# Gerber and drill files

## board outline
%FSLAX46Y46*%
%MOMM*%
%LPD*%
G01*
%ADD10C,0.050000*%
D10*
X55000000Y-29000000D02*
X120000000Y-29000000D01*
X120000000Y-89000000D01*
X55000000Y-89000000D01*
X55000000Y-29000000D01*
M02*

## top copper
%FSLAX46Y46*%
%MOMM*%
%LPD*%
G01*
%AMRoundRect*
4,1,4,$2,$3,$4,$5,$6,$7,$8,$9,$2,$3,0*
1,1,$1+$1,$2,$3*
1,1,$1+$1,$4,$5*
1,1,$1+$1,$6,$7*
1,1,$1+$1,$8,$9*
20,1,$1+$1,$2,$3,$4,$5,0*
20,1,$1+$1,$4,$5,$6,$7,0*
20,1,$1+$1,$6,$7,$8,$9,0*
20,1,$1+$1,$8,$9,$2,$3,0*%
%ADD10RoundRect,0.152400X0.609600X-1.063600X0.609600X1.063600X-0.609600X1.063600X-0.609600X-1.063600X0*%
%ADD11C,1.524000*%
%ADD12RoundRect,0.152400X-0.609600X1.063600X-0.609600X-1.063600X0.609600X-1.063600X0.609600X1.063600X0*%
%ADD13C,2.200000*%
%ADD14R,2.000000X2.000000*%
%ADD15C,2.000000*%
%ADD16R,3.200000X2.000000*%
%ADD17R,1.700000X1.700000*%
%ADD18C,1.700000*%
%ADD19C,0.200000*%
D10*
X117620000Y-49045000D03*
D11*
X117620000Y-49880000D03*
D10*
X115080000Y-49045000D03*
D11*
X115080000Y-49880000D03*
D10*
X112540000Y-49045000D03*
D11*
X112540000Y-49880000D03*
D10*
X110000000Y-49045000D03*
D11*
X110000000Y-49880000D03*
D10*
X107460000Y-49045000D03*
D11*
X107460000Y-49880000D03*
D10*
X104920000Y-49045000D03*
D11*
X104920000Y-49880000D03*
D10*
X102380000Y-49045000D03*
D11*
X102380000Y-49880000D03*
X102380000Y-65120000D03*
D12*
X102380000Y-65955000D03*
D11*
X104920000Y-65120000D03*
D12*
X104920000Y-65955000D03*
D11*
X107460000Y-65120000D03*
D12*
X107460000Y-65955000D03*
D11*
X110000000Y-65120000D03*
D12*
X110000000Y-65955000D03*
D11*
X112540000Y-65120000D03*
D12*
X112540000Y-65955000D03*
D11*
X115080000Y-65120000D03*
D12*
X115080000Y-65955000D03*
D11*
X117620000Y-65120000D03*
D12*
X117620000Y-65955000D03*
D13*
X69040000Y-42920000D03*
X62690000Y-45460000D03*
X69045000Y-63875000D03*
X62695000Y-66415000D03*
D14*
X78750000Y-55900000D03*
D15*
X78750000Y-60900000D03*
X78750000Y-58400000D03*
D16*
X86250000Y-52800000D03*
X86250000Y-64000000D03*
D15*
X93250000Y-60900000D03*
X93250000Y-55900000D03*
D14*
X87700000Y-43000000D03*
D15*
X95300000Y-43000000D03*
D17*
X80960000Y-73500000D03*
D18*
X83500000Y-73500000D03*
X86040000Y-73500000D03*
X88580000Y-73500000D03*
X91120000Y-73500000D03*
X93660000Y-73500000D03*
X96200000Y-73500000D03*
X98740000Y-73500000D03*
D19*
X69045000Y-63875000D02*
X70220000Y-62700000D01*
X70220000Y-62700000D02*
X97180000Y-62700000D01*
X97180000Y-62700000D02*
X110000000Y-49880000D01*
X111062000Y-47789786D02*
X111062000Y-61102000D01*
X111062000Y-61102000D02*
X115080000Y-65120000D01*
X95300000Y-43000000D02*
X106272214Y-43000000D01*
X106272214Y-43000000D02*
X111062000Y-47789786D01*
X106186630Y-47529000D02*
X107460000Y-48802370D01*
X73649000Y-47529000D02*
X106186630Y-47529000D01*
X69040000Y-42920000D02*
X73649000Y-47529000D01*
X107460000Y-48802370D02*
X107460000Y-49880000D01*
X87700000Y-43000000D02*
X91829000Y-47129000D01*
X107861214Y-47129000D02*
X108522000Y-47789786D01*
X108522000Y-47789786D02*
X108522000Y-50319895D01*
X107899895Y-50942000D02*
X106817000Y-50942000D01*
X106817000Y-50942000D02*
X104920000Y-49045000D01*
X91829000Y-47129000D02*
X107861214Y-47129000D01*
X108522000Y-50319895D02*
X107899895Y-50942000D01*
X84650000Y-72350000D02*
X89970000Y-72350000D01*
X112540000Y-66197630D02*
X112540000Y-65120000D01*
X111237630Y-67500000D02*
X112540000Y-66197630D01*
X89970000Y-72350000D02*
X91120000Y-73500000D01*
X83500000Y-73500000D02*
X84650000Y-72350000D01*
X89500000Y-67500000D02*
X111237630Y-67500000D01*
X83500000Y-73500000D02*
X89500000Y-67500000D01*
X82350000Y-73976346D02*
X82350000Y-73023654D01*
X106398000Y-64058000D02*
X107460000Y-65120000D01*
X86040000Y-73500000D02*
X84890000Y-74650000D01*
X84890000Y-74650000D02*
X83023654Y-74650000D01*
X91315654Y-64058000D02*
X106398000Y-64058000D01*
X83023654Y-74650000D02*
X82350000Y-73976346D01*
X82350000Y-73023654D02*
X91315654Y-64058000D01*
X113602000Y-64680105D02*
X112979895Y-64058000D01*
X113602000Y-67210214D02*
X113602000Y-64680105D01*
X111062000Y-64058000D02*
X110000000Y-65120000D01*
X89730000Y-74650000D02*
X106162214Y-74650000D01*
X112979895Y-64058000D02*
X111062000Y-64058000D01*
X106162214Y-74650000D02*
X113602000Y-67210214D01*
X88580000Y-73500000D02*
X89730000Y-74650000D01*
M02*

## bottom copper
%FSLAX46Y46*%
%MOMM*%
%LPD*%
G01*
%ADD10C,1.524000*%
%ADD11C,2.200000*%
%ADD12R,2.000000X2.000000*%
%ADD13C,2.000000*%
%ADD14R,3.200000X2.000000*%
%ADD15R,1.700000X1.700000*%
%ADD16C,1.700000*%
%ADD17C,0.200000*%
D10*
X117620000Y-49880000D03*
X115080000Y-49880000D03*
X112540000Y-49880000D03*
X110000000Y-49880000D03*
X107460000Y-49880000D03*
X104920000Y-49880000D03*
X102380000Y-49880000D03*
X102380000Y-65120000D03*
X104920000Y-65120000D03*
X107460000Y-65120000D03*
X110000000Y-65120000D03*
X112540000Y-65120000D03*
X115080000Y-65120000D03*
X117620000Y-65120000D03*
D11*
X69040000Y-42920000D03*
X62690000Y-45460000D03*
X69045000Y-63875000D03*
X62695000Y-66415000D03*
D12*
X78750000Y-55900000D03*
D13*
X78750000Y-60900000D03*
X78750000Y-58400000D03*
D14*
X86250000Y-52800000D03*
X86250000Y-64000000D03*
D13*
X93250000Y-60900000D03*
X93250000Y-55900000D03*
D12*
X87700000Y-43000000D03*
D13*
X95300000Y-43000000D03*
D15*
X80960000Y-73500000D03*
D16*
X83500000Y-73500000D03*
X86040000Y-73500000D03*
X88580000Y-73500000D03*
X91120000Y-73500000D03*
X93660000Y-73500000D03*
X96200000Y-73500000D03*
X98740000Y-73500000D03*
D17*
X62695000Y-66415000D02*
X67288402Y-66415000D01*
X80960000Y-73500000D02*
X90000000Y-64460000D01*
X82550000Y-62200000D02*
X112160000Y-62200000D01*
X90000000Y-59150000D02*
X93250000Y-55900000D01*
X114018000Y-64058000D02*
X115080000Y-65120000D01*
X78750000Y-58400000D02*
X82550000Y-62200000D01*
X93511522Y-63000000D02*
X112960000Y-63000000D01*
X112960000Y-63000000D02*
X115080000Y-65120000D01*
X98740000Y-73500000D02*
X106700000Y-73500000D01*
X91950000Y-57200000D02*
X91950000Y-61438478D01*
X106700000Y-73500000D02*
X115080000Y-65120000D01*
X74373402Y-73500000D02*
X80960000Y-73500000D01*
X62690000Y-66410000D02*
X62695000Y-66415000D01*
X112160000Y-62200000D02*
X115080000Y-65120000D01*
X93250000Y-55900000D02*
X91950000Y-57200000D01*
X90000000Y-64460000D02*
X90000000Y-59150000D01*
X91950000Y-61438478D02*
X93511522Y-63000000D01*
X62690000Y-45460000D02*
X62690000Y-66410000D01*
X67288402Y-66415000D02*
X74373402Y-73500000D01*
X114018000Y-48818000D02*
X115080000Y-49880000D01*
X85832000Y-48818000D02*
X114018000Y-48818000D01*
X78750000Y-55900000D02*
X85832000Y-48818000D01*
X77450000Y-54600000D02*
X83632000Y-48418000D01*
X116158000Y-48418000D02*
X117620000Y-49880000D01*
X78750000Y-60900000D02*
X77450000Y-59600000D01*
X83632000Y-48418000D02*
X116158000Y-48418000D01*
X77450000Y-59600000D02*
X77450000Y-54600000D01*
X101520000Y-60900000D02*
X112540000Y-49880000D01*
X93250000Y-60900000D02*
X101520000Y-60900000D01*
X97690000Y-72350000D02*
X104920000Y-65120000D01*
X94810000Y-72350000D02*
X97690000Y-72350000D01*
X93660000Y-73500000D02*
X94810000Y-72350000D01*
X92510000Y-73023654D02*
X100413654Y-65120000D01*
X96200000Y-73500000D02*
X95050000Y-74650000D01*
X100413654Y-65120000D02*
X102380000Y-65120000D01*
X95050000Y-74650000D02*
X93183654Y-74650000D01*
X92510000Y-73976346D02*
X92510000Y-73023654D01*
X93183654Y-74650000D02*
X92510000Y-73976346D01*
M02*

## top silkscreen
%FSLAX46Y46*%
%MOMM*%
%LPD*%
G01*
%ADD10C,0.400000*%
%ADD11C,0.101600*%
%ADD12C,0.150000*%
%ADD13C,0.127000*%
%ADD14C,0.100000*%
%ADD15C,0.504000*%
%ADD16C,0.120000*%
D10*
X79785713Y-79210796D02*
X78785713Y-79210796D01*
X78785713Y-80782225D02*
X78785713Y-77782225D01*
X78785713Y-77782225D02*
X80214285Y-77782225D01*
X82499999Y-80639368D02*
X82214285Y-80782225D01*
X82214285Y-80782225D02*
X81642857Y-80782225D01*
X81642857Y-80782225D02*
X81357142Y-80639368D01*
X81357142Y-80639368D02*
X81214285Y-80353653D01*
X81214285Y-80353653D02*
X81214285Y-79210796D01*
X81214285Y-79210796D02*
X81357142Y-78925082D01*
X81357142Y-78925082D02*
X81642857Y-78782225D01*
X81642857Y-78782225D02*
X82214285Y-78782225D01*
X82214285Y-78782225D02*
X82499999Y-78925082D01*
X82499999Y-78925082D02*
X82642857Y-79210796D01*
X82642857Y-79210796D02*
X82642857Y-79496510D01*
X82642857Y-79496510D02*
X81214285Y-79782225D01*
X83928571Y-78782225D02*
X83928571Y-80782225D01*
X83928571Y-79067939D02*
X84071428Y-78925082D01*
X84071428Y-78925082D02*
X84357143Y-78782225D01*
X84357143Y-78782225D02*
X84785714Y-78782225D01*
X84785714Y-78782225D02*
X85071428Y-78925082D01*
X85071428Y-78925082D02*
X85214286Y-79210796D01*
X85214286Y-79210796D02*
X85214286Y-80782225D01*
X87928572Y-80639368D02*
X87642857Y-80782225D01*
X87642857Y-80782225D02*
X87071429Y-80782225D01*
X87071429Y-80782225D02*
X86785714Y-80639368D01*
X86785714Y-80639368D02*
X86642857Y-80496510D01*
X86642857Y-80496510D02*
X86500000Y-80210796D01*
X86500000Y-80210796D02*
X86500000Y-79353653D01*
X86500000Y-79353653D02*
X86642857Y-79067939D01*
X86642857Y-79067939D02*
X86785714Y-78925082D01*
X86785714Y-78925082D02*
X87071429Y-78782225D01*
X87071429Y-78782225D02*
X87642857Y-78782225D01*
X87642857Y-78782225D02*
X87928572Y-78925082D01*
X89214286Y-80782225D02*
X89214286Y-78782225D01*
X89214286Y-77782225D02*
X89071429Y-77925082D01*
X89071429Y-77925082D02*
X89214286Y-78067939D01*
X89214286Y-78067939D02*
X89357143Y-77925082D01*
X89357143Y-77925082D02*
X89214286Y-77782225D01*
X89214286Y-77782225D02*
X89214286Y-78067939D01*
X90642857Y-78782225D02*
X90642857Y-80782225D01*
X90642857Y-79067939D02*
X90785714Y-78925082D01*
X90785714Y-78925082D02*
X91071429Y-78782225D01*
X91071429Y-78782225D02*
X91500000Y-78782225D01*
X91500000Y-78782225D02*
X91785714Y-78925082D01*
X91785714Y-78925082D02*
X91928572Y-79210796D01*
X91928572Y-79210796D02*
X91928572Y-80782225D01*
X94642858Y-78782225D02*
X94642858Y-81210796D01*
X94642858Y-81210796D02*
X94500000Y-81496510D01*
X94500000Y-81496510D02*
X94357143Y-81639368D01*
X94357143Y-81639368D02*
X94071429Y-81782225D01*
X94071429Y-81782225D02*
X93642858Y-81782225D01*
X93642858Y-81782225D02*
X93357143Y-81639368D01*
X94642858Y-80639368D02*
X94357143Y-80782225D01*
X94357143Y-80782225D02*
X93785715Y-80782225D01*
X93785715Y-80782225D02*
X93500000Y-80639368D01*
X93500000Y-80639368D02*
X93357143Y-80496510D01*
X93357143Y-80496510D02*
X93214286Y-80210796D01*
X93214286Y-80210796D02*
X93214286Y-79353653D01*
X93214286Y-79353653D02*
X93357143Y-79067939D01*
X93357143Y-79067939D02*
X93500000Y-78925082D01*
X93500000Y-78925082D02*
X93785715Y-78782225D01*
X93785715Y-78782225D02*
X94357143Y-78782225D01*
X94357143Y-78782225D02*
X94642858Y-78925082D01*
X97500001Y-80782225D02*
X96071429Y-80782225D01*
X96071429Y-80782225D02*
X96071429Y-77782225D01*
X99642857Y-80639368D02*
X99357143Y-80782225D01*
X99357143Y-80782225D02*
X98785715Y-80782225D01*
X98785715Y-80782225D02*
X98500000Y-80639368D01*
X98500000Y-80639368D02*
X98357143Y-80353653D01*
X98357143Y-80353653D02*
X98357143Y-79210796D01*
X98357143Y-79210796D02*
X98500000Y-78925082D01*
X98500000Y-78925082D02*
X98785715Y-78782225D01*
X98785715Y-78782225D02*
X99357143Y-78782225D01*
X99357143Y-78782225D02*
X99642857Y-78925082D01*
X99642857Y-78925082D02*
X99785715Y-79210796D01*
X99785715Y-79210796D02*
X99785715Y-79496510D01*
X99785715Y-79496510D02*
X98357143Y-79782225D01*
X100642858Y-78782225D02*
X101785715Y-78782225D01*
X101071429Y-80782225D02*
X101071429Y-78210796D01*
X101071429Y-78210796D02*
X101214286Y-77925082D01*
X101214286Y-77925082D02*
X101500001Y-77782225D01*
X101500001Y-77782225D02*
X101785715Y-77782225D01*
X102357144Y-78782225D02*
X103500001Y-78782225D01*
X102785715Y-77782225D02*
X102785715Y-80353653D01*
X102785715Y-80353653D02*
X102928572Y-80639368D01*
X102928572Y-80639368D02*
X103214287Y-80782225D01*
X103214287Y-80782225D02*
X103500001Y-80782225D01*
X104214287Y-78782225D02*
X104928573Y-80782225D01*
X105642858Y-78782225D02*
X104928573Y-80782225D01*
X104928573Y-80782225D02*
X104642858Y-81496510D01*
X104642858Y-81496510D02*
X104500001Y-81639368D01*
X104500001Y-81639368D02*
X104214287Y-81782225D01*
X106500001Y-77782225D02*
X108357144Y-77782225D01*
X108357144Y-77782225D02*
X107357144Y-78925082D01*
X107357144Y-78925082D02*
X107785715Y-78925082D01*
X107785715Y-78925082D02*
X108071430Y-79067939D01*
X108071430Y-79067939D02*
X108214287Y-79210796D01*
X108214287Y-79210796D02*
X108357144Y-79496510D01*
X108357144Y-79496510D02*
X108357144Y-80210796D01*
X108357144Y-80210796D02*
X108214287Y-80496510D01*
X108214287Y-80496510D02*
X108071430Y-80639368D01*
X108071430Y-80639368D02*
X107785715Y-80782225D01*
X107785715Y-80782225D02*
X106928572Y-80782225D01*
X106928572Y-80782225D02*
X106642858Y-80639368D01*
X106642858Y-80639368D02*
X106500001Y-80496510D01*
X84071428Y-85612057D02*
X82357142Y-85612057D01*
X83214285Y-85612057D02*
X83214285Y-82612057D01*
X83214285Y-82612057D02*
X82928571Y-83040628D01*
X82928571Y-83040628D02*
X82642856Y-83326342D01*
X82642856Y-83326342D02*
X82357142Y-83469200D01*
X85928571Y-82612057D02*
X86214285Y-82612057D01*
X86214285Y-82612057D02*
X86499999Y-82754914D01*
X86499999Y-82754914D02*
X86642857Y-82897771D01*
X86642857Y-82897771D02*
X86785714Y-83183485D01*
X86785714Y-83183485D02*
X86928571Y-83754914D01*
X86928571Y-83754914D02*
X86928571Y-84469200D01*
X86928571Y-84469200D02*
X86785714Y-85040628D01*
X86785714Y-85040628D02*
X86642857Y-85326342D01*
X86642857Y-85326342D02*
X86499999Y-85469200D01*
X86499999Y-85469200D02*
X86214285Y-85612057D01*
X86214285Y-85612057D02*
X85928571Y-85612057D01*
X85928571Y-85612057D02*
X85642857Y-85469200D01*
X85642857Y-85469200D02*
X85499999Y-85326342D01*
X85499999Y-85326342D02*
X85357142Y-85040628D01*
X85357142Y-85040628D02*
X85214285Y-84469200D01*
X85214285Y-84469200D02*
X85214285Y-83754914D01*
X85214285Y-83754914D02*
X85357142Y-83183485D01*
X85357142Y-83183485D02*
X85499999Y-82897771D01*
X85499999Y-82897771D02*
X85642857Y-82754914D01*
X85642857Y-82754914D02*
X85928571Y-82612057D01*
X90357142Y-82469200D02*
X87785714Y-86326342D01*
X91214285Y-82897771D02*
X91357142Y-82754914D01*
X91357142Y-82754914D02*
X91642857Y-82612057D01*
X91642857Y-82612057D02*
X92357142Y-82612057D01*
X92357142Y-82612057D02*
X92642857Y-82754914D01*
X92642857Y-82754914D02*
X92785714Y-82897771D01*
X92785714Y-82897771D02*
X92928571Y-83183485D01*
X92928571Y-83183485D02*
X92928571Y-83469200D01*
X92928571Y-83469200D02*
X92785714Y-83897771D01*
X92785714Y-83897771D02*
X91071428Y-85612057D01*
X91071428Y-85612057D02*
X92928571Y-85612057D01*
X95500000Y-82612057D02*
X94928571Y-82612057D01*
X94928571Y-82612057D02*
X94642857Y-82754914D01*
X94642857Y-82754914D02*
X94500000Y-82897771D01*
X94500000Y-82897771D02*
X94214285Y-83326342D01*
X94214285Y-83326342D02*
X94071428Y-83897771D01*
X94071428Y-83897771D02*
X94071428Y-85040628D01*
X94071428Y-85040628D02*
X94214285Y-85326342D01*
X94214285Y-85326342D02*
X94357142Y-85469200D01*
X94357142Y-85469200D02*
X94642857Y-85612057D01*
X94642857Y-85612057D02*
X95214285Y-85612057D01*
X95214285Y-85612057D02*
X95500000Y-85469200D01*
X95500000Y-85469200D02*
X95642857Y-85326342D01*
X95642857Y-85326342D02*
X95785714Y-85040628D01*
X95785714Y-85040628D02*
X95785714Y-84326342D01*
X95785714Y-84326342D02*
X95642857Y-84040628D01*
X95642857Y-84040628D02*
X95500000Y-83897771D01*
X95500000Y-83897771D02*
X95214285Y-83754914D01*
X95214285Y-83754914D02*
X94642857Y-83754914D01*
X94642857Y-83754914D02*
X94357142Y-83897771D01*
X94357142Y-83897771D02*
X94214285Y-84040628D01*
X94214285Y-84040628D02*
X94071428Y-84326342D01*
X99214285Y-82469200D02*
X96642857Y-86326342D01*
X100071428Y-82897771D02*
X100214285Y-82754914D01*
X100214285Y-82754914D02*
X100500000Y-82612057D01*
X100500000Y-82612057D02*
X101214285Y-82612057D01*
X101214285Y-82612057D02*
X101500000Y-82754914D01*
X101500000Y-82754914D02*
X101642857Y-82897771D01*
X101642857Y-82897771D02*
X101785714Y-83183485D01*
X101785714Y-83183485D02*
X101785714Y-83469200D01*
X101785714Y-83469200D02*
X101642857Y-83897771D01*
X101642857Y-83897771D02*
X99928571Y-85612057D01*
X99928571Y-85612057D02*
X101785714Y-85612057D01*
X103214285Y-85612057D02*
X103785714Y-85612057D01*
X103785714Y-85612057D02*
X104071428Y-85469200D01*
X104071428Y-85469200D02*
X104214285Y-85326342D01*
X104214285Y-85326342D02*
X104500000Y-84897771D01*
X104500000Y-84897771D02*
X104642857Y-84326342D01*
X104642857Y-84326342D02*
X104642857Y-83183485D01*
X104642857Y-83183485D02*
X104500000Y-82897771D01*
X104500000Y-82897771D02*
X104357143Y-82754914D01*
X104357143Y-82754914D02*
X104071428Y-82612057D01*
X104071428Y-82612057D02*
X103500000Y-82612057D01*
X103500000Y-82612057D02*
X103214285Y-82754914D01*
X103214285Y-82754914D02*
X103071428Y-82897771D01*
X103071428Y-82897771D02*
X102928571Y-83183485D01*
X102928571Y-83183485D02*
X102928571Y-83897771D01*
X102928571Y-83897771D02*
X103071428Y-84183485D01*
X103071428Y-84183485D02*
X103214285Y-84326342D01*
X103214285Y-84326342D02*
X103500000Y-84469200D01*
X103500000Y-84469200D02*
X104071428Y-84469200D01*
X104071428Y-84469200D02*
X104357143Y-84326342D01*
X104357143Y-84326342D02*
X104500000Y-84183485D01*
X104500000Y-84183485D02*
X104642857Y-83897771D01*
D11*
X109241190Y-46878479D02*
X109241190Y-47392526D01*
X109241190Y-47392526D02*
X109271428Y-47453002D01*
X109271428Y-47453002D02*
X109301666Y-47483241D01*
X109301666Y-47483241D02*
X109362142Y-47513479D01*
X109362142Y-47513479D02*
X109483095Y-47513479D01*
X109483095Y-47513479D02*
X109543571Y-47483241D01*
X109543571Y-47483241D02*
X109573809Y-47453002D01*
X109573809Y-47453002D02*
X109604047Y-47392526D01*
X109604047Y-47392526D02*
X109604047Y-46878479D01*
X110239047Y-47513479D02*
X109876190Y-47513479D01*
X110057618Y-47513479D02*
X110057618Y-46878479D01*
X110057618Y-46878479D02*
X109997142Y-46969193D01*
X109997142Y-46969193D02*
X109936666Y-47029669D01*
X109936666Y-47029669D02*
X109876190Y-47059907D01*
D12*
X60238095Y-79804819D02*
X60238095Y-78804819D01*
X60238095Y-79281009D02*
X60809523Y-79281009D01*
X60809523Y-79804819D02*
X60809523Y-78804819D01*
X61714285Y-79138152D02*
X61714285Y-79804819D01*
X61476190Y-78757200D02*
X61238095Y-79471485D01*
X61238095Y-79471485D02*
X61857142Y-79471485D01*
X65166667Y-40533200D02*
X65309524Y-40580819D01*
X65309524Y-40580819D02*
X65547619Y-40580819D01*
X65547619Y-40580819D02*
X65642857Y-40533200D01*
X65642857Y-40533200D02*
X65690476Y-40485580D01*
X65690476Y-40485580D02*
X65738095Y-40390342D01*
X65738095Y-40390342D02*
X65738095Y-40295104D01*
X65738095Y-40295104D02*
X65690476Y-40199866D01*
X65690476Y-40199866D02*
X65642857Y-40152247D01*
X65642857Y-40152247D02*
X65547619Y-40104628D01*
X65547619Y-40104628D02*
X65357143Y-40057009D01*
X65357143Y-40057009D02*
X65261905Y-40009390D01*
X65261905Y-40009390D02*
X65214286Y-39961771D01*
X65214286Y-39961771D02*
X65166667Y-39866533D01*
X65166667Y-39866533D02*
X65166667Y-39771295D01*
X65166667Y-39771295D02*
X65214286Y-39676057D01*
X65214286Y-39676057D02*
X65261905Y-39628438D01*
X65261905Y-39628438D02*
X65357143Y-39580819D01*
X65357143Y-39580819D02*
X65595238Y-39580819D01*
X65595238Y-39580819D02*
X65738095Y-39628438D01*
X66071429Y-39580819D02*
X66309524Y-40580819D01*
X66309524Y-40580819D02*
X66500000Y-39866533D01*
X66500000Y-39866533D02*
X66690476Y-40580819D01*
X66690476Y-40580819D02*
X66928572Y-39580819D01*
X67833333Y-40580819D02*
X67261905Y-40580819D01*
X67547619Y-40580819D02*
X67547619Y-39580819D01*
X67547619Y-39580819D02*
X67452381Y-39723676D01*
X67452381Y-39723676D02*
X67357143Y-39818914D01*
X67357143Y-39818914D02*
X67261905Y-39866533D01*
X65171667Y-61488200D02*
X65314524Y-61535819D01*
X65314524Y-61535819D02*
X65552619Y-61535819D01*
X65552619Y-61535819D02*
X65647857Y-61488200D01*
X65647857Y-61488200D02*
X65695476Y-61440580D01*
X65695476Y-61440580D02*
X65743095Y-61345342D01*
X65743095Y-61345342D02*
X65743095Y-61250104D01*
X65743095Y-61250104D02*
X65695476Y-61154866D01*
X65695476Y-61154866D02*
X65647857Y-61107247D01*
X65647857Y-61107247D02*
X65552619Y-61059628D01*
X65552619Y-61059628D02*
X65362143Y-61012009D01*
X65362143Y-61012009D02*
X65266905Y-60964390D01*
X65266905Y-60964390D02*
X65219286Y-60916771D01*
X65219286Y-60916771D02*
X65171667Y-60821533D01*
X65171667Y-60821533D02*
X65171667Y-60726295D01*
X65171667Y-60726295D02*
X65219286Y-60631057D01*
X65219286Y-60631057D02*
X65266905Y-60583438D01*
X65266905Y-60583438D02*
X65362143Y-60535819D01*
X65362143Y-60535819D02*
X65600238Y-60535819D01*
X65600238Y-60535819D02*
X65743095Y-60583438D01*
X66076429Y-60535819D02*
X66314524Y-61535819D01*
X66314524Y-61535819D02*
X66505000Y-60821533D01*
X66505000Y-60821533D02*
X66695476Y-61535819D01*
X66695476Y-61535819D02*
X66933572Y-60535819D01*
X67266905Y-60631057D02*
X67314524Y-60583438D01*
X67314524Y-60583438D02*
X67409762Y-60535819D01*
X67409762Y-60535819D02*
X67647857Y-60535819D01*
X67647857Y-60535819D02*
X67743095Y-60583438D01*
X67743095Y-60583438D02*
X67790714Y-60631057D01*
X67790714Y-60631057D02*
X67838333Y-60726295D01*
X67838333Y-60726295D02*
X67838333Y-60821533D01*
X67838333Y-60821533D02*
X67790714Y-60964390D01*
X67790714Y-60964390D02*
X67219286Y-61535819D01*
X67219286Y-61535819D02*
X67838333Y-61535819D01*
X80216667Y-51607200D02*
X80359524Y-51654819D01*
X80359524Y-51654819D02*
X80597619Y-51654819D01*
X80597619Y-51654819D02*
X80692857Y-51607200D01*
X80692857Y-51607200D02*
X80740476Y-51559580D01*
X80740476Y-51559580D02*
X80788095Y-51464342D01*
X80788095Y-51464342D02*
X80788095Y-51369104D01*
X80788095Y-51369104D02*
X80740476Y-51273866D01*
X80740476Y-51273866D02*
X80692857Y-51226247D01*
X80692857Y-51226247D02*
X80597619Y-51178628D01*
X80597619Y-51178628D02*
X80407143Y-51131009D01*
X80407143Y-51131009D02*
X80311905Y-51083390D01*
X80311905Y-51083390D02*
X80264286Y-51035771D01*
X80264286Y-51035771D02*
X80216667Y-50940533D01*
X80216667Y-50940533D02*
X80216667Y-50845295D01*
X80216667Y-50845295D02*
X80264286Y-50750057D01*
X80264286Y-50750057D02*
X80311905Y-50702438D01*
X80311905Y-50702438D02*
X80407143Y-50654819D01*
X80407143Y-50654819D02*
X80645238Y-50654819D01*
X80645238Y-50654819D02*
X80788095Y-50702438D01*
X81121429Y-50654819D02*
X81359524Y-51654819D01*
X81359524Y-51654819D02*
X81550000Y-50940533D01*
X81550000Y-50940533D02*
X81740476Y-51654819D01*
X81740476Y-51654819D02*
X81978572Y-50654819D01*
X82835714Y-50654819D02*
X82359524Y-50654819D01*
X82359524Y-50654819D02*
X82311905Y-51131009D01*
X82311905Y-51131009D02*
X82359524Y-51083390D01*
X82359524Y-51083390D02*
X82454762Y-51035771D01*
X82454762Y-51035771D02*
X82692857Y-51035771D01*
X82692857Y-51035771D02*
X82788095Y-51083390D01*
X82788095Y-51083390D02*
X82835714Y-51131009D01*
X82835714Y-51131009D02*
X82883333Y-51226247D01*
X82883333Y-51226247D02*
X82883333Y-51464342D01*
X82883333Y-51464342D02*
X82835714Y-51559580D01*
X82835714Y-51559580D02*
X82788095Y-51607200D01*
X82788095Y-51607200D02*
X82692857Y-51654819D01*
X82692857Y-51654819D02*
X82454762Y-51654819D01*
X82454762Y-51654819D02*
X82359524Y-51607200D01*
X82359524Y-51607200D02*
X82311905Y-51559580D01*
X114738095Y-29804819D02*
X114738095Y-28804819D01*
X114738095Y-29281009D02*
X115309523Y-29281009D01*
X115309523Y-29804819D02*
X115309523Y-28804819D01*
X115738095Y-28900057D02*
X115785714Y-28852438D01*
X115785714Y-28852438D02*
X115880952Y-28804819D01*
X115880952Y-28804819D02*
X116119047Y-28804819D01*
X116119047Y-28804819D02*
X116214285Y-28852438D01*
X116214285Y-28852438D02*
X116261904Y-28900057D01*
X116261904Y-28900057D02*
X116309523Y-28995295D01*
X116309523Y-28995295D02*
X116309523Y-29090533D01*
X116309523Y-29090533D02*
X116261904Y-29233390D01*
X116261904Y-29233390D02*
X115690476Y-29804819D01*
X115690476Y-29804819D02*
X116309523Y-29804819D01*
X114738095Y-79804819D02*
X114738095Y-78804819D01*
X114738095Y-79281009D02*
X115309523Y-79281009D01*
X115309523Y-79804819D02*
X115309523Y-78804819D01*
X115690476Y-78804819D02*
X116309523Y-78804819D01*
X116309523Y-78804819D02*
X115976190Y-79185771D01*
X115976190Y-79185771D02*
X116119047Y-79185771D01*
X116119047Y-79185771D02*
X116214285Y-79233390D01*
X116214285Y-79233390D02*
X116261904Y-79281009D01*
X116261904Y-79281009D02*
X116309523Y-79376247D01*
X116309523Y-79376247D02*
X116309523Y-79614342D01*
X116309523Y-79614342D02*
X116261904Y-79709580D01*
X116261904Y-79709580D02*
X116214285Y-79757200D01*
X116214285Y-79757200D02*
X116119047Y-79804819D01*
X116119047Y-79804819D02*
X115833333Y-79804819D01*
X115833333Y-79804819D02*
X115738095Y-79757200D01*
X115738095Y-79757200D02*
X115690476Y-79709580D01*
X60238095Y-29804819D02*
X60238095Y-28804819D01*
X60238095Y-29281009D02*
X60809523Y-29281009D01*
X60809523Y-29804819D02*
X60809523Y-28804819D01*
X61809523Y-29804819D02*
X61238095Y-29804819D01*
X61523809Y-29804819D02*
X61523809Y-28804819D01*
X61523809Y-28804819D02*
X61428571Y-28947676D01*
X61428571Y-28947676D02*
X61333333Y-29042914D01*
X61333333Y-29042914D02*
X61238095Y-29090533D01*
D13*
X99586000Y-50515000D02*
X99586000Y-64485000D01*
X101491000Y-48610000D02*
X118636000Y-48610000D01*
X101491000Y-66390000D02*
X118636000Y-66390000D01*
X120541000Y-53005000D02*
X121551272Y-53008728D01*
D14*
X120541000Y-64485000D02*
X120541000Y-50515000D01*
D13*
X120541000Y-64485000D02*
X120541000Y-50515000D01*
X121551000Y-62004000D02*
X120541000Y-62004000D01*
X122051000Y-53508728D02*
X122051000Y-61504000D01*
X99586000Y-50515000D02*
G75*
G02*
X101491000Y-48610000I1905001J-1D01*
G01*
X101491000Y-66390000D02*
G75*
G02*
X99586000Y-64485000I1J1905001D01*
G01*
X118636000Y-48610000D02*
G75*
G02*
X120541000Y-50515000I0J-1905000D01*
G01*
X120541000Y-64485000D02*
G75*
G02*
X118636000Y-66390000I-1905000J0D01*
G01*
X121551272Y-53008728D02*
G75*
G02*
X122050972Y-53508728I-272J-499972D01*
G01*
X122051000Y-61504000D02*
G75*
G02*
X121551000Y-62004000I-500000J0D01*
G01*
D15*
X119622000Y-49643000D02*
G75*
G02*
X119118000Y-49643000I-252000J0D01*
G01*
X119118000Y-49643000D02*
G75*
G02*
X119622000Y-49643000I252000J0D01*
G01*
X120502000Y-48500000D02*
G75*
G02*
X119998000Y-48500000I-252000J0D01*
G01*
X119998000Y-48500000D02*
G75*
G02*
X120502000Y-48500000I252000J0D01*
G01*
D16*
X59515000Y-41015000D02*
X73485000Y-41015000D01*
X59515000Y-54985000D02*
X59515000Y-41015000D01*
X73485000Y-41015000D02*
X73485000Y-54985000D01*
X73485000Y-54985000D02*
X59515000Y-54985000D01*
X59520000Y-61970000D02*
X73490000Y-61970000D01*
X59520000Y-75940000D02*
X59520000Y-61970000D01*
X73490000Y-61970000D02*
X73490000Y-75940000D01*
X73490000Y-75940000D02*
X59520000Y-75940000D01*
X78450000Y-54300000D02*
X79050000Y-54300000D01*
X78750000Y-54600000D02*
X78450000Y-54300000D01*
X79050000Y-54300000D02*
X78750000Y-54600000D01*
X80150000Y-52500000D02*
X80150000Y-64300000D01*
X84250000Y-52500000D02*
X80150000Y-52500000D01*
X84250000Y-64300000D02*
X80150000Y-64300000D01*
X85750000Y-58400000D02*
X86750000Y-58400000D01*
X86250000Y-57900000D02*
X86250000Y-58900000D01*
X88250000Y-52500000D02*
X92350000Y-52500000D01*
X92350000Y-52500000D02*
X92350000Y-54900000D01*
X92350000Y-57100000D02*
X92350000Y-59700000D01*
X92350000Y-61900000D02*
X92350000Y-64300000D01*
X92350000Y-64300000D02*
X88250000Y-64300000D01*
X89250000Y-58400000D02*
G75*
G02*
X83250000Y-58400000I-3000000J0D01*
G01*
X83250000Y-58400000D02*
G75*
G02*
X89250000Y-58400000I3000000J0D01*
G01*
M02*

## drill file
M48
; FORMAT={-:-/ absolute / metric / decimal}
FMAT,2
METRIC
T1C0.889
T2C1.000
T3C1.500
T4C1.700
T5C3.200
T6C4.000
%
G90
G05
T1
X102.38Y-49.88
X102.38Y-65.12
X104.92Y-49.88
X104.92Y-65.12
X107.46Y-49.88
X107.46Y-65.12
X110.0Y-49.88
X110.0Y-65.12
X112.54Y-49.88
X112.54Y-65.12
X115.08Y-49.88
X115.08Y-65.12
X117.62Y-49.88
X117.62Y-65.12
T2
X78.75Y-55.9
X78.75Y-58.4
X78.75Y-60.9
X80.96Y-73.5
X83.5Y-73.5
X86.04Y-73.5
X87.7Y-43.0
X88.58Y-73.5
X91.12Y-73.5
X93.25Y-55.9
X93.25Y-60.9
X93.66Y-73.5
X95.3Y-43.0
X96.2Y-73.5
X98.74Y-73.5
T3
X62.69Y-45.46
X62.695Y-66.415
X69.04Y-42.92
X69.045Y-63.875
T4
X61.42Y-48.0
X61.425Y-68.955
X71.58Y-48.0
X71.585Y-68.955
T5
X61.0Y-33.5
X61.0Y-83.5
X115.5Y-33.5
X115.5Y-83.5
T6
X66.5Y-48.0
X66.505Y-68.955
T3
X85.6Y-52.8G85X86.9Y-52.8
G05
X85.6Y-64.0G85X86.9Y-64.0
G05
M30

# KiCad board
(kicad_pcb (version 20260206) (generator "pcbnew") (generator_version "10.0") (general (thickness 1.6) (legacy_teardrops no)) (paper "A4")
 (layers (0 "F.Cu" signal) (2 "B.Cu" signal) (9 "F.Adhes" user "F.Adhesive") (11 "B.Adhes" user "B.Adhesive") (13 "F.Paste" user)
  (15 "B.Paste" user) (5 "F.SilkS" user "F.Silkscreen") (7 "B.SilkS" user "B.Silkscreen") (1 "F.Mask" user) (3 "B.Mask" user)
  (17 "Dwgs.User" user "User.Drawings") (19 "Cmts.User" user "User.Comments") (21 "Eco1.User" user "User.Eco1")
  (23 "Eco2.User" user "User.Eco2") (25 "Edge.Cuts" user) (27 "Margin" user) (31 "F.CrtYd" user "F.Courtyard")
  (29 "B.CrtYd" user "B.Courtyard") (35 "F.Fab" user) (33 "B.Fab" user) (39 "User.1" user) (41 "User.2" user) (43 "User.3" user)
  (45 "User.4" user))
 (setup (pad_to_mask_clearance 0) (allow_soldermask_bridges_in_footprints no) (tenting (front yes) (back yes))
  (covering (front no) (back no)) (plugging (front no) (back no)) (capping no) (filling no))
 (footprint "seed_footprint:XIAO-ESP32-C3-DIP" (layer "F.Cu") (at 110 57.5)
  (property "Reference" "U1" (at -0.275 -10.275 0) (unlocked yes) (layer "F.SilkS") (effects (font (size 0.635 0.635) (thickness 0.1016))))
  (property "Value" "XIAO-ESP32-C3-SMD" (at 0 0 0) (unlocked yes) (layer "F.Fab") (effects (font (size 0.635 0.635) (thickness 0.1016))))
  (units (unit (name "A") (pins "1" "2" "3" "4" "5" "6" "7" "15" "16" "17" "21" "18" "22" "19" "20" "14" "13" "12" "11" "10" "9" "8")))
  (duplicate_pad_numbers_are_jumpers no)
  (fp_line (start -10.414 -6.985) (end -10.414 6.985) (stroke (width 0.127) (type solid)) (layer "F.SilkS"))
  (fp_line (start -8.509 -8.89) (end 8.636 -8.89) (stroke (width 0.127) (type solid)) (layer "F.SilkS"))
  (fp_line (start -8.509 8.89) (end 8.636 8.89) (stroke (width 0.127) (type solid)) (layer "F.SilkS"))
  (fp_line (start 10.541 -4.495) (end 11.551272 -4.491272) (stroke (width 0.127) (type solid)) (layer "F.SilkS"))
  (fp_line (start 10.541 6.985) (end 10.541 -6.985) (stroke (width 0.1) (type solid)) (layer "F.SilkS"))
  (fp_line (start 10.541 6.985) (end 10.541 -6.985) (stroke (width 0.127) (type solid)) (layer "F.SilkS"))
  (fp_line (start 11.551 4.504) (end 10.541 4.504) (stroke (width 0.127) (type solid)) (layer "F.SilkS"))
  (fp_line (start 12.051 -3.991272) (end 12.051 4.004) (stroke (width 0.127) (type solid)) (layer "F.SilkS"))
  (fp_arc (start -10.414 -6.985) (mid -9.856038 -8.332038) (end -8.509 -8.89) (stroke (width 0.127) (type solid)) (layer "F.SilkS"))
  (fp_arc (start -8.509 8.89) (mid -9.856038 8.332038) (end -10.414 6.985) (stroke (width 0.127) (type solid)) (layer "F.SilkS"))
  (fp_arc (start 8.636 -8.89) (mid 9.983038 -8.332038) (end 10.541 -6.985) (stroke (width 0.127) (type solid)) (layer "F.SilkS"))
  (fp_arc (start 10.541 6.985) (mid 9.983038 8.332038) (end 8.636 8.89) (stroke (width 0.127) (type solid)) (layer "F.SilkS"))
  (fp_arc (start 11.551272 -4.491272) (mid 11.904644 -4.344724) (end 12.051 -3.991272) (stroke (width 0.127) (type default))
   (layer "F.SilkS"))
  (fp_arc (start 12.051 4.004) (mid 11.904553 4.357553) (end 11.551 4.504) (stroke (width 0.127) (type default)) (layer "F.SilkS"))
  (fp_circle (center 9.37 -7.857) (end 9.624 -7.857) (stroke (width 0.5) (type solid)) (fill yes) (layer "F.SilkS"))
  (fp_circle (center 10.25 -9) (end 10.504 -9) (stroke (width 0.5) (type solid)) (fill yes) (layer "F.SilkS"))
  (pad "1" smd roundrect (at 7.62 -8.455 90) (size 2.432 1.524) (layers "F.Cu" "F.Mask") (roundrect_rratio 0.1) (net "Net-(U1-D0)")
   (thermal_bridge_angle 45))
  (pad "1" thru_hole circle (at 7.62 -7.62 90) (size 1.524 1.524) (drill 0.889) (layers "*.Cu" "*.Mask") (remove_unused_layers no)
   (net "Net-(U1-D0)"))
  (pad "2" smd roundrect (at 5.08 -8.455 90) (size 2.432 1.524) (layers "F.Cu" "F.Mask") (roundrect_rratio 0.1) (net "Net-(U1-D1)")
   (thermal_bridge_angle 45))
  (pad "2" thru_hole circle (at 5.08 -7.62 90) (size 1.524 1.524) (drill 0.889) (layers "*.Cu" "*.Mask") (remove_unused_layers no)
   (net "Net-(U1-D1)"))
  (pad "3" smd roundrect (at 2.54 -8.455 90) (size 2.432 1.524) (layers "F.Cu" "F.Mask") (roundrect_rratio 0.1) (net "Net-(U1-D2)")
   (thermal_bridge_angle 45))
  (pad "3" thru_hole circle (at 2.54 -7.62 90) (size 1.524 1.524) (drill 0.889) (layers "*.Cu" "*.Mask") (remove_unused_layers no)
   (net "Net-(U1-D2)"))
  (pad "4" smd roundrect (at 0 -8.455 90) (size 2.432 1.524) (layers "F.Cu" "F.Mask") (roundrect_rratio 0.1) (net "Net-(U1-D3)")
   (thermal_bridge_angle 45))
  (pad "4" thru_hole circle (at 0 -7.62 90) (size 1.524 1.524) (drill 0.889) (layers "*.Cu" "*.Mask") (remove_unused_layers no)
   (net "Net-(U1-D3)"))
  (pad "5" smd roundrect (at -2.54 -8.455 90) (size 2.432 1.524) (layers "F.Cu" "F.Mask") (roundrect_rratio 0.1) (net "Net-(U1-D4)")
   (thermal_bridge_angle 45))
  (pad "5" thru_hole circle (at -2.54 -7.62 90) (size 1.524 1.524) (drill 0.889) (layers "*.Cu" "*.Mask") (remove_unused_layers no)
   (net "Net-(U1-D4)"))
  (pad "6" smd roundrect (at -5.08 -8.455 90) (size 2.432 1.524) (layers "F.Cu" "F.Mask") (roundrect_rratio 0.1) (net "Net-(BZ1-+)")
   (thermal_bridge_angle 45))
  (pad "6" thru_hole circle (at -5.08 -7.62 90) (size 1.524 1.524) (drill 0.889) (layers "*.Cu" "*.Mask") (remove_unused_layers no)
   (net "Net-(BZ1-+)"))
  (pad "7" smd roundrect (at -7.62 -8.455 90) (size 2.432 1.524) (layers "F.Cu" "F.Mask") (roundrect_rratio 0.1)
   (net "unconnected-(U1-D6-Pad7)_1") (thermal_bridge_angle 45))
  (pad "7" thru_hole circle (at -7.62 -7.62 90) (size 1.524 1.524) (drill 0.889) (layers "*.Cu" "*.Mask") (remove_unused_layers no)
   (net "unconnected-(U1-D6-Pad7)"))
  (pad "8" thru_hole circle (at -7.62 7.62 270) (size 1.524 1.524) (drill 0.889) (layers "*.Cu" "*.Mask") (remove_unused_layers no)
   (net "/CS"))
  (pad "8" smd roundrect (at -7.62 8.455 270) (size 2.432 1.524) (layers "F.Cu" "F.Mask") (roundrect_rratio 0.1) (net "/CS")
   (thermal_bridge_angle 45))
  (pad "9" thru_hole circle (at -5.08 7.62 270) (size 1.524 1.524) (drill 0.889) (layers "*.Cu" "*.Mask") (remove_unused_layers no)
   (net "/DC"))
  (pad "9" smd roundrect (at -5.08 8.455 270) (size 2.432 1.524) (layers "F.Cu" "F.Mask") (roundrect_rratio 0.1) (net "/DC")
   (thermal_bridge_angle 45))
  (pad "10" thru_hole circle (at -2.54 7.62 270) (size 1.524 1.524) (drill 0.889) (layers "*.Cu" "*.Mask") (remove_unused_layers no)
   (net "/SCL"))
  (pad "10" smd roundrect (at -2.54 8.455 270) (size 2.432 1.524) (layers "F.Cu" "F.Mask") (roundrect_rratio 0.1) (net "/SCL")
   (thermal_bridge_angle 45))
  (pad "11" thru_hole circle (at 0 7.62 270) (size 1.524 1.524) (drill 0.889) (layers "*.Cu" "*.Mask") (remove_unused_layers no)
   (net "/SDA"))
  (pad "11" smd roundrect (at 0 8.455 270) (size 2.432 1.524) (layers "F.Cu" "F.Mask") (roundrect_rratio 0.1) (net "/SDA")
   (thermal_bridge_angle 45))
  (pad "12" thru_hole circle (at 2.54 7.62 270) (size 1.524 1.524) (drill 0.889) (layers "*.Cu" "*.Mask") (remove_unused_layers no)
   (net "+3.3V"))
  (pad "12" smd roundrect (at 2.54 8.455 270) (size 2.432 1.524) (layers "F.Cu" "F.Mask") (roundrect_rratio 0.1) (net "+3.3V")
   (thermal_bridge_angle 45))
  (pad "13" thru_hole circle (at 5.08 7.62 270) (size 1.524 1.524) (drill 0.889) (layers "*.Cu" "*.Mask") (remove_unused_layers no)
   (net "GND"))
  (pad "13" smd roundrect (at 5.08 8.455 270) (size 2.432 1.524) (layers "F.Cu" "F.Mask") (roundrect_rratio 0.1) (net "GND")
   (thermal_bridge_angle 45))
  (pad "14" thru_hole circle (at 7.62 7.62 270) (size 1.524 1.524) (drill 0.889) (layers "*.Cu" "*.Mask") (remove_unused_layers no)
   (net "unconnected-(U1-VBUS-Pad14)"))
  (pad "14" smd roundrect (at 7.62 8.455 270) (size 2.432 1.524) (layers "F.Cu" "F.Mask") (roundrect_rratio 0.1)
   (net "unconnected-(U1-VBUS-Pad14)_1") (thermal_bridge_angle 45)))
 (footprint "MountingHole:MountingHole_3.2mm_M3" (layer "F.Cu") (at 61 83.5)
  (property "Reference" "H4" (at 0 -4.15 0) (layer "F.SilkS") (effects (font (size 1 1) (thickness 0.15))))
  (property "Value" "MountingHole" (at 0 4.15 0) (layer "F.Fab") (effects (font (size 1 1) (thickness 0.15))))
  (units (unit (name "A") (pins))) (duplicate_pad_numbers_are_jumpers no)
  (pad "" np_thru_hole circle (at 0 0) (size 3.2 3.2) (drill 3.2) (layers "*.Cu" "*.Mask")))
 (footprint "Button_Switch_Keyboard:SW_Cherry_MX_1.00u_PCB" (layer "F.Cu") (at 69.04 42.92)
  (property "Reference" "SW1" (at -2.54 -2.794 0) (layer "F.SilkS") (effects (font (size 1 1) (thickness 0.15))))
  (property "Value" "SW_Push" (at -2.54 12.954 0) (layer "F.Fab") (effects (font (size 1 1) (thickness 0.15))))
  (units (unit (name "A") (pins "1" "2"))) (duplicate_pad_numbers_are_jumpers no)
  (fp_line (start -9.525 -1.905) (end 4.445 -1.905) (stroke (width 0.12) (type solid)) (layer "F.SilkS"))
  (fp_line (start -9.525 12.065) (end -9.525 -1.905) (stroke (width 0.12) (type solid)) (layer "F.SilkS"))
  (fp_line (start 4.445 -1.905) (end 4.445 12.065) (stroke (width 0.12) (type solid)) (layer "F.SilkS"))
  (fp_line (start 4.445 12.065) (end -9.525 12.065) (stroke (width 0.12) (type solid)) (layer "F.SilkS"))
  (pad "" np_thru_hole circle (at -7.62 5.08) (size 1.7 1.7) (drill 1.7) (layers "*.Cu" "*.Mask"))
  (pad "" np_thru_hole circle (at -2.54 5.08) (size 4 4) (drill 4) (layers "*.Cu" "*.Mask"))
  (pad "" np_thru_hole circle (at 2.54 5.08) (size 1.7 1.7) (drill 1.7) (layers "*.Cu" "*.Mask"))
  (pad "1" thru_hole circle (at 0 0) (size 2.2 2.2) (drill 1.5) (layers "*.Cu" "*.Mask") (remove_unused_layers no) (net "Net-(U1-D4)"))
  (pad "2" thru_hole circle (at -6.35 2.54) (size 2.2 2.2) (drill 1.5) (layers "*.Cu" "*.Mask") (remove_unused_layers no) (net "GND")))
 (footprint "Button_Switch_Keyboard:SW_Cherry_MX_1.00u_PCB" (layer "F.Cu") (at 69.045 63.875)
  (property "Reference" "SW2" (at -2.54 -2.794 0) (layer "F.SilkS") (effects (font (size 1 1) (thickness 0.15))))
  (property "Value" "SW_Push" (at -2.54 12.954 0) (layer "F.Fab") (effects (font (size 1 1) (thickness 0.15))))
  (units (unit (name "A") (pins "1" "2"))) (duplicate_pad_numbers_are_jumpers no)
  (fp_line (start -9.525 -1.905) (end 4.445 -1.905) (stroke (width 0.12) (type solid)) (layer "F.SilkS"))
  (fp_line (start -9.525 12.065) (end -9.525 -1.905) (stroke (width 0.12) (type solid)) (layer "F.SilkS"))
  (fp_line (start 4.445 -1.905) (end 4.445 12.065) (stroke (width 0.12) (type solid)) (layer "F.SilkS"))
  (fp_line (start 4.445 12.065) (end -9.525 12.065) (stroke (width 0.12) (type solid)) (layer "F.SilkS"))
  (pad "" np_thru_hole circle (at -7.62 5.08) (size 1.7 1.7) (drill 1.7) (layers "*.Cu" "*.Mask"))
  (pad "" np_thru_hole circle (at -2.54 5.08) (size 4 4) (drill 4) (layers "*.Cu" "*.Mask"))
  (pad "" np_thru_hole circle (at 2.54 5.08) (size 1.7 1.7) (drill 1.7) (layers "*.Cu" "*.Mask"))
  (pad "1" thru_hole circle (at 0 0) (size 2.2 2.2) (drill 1.5) (layers "*.Cu" "*.Mask") (remove_unused_layers no) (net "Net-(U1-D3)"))
  (pad "2" thru_hole circle (at -6.35 2.54) (size 2.2 2.2) (drill 1.5) (layers "*.Cu" "*.Mask") (remove_unused_layers no) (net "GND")))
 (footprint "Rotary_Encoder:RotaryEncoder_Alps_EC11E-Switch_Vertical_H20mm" (layer "F.Cu") (at 78.75 55.9)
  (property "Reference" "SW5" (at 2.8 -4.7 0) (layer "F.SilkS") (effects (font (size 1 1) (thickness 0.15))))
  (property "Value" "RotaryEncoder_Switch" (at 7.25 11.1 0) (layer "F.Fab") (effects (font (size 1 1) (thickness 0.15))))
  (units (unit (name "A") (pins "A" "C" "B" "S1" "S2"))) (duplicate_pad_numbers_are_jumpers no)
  (fp_line (start -0.3 -1.6) (end 0.3 -1.6) (stroke (width 0.12) (type solid)) (layer "F.SilkS"))
  (fp_line (start 0 -1.3) (end -0.3 -1.6) (stroke (width 0.12) (type solid)) (layer "F.SilkS"))
  (fp_line (start 0.3 -1.6) (end 0 -1.3) (stroke (width 0.12) (type solid)) (layer "F.SilkS"))
  (fp_line (start 1.4 -3.4) (end 1.4 8.4) (stroke (width 0.12) (type solid)) (layer "F.SilkS"))
  (fp_line (start 5.5 -3.4) (end 1.4 -3.4) (stroke (width 0.12) (type solid)) (layer "F.SilkS"))
  (fp_line (start 5.5 8.4) (end 1.4 8.4) (stroke (width 0.12) (type solid)) (layer "F.SilkS"))
  (fp_line (start 7 2.5) (end 8 2.5) (stroke (width 0.12) (type solid)) (layer "F.SilkS"))
  (fp_line (start 7.5 2) (end 7.5 3) (stroke (width 0.12) (type solid)) (layer "F.SilkS"))
  (fp_line (start 9.5 -3.4) (end 13.6 -3.4) (stroke (width 0.12) (type solid)) (layer "F.SilkS"))
  (fp_line (start 13.6 -3.4) (end 13.6 -1) (stroke (width 0.12) (type solid)) (layer "F.SilkS"))
  (fp_line (start 13.6 1.2) (end 13.6 3.8) (stroke (width 0.12) (type solid)) (layer "F.SilkS"))
  (fp_line (start 13.6 6) (end 13.6 8.4) (stroke (width 0.12) (type solid)) (layer "F.SilkS"))
  (fp_line (start 13.6 8.4) (end 9.5 8.4) (stroke (width 0.12) (type solid)) (layer "F.SilkS"))
  (fp_circle (center 7.5 2.5) (end 10.5 2.5) (stroke (width 0.12) (type solid)) (fill no) (layer "F.SilkS"))
  (pad "A" thru_hole rect (at 0 0) (size 2 2) (drill 1) (layers "*.Cu" "*.Mask") (remove_unused_layers no) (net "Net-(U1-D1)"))
  (pad "B" thru_hole circle (at 0 5) (size 2 2) (drill 1) (layers "*.Cu" "*.Mask") (remove_unused_layers no) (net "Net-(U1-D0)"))
  (pad "C" thru_hole circle (at 0 2.5) (size 2 2) (drill 1) (layers "*.Cu" "*.Mask") (remove_unused_layers no) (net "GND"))
  (pad "MP" thru_hole rect (at 7.5 -3.1) (size 3.2 2) (drill oval 2.8 1.5) (layers "*.Cu" "*.Mask") (remove_unused_layers no))
  (pad "MP" thru_hole rect (at 7.5 8.1) (size 3.2 2) (drill oval 2.8 1.5) (layers "*.Cu" "*.Mask") (remove_unused_layers no))
  (pad "S1" thru_hole circle (at 14.5 5) (size 2 2) (drill 1) (layers "*.Cu" "*.Mask") (remove_unused_layers no) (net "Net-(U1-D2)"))
  (pad "S2" thru_hole circle (at 14.5 0) (size 2 2) (drill 1) (layers "*.Cu" "*.Mask") (remove_unused_layers no) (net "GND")))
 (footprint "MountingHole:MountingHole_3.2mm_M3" (layer "F.Cu") (at 115.5 33.5)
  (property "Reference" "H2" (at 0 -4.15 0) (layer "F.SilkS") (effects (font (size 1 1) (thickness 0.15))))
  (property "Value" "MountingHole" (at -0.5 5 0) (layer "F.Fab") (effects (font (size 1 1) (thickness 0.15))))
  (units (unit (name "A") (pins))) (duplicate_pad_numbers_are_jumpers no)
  (pad "" np_thru_hole circle (at 0 0) (size 3.2 3.2) (drill 3.2) (layers "*.Cu" "*.Mask")))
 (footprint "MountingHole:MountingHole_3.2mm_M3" (layer "F.Cu") (at 115.5 83.5)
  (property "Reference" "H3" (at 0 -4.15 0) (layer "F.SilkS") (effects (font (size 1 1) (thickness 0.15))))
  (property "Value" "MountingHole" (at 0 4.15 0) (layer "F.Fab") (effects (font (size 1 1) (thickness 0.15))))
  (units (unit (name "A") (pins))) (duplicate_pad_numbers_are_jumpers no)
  (pad "" np_thru_hole circle (at 0 0) (size 3.2 3.2) (drill 3.2) (layers "*.Cu" "*.Mask")))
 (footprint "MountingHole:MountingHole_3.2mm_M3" (layer "F.Cu") (at 61 33.5)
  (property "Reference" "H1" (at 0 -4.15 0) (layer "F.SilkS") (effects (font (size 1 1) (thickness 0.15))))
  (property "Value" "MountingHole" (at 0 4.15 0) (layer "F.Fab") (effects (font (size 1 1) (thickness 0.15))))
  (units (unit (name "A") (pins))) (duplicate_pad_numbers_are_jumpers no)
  (pad "" np_thru_hole circle (at 0 0) (size 3.2 3.2) (drill 3.2) (layers "*.Cu" "*.Mask")))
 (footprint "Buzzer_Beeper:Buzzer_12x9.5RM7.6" (layer "B.Cu") (at 87.7 43)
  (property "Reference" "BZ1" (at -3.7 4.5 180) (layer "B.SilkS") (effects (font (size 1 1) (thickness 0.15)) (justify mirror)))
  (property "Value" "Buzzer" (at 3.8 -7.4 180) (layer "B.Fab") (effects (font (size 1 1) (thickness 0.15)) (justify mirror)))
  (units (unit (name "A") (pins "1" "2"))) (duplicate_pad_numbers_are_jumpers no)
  (pad "1" thru_hole rect (at 0 0) (size 2 2) (drill 1) (layers "*.Cu" "*.Mask") (remove_unused_layers no) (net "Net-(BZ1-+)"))
  (pad "2" thru_hole circle (at 7.6 0) (size 2 2) (drill 1) (layers "*.Cu" "*.Mask") (remove_unused_layers no) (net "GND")))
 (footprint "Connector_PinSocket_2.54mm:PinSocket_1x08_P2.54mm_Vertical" (layer "B.Cu") (at 80.96 73.5 -90)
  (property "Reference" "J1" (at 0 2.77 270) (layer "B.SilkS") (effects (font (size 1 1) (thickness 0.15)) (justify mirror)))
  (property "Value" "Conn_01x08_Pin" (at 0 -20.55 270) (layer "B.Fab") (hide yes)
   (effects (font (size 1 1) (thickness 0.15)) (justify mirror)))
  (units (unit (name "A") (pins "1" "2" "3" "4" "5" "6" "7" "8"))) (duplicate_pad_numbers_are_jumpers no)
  (pad "1" thru_hole rect (at 0 0 270) (size 1.7 1.7) (drill 1) (layers "*.Cu" "*.Mask") (remove_unused_layers no) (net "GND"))
  (pad "2" thru_hole circle (at 0 -2.54 270) (size 1.7 1.7) (drill 1) (layers "*.Cu" "*.Mask") (remove_unused_layers no) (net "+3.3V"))
  (pad "3" thru_hole circle (at 0 -5.08 270) (size 1.7 1.7) (drill 1) (layers "*.Cu" "*.Mask") (remove_unused_layers no) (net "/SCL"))
  (pad "4" thru_hole circle (at 0 -7.62 270) (size 1.7 1.7) (drill 1) (layers "*.Cu" "*.Mask") (remove_unused_layers no) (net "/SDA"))
  (pad "5" thru_hole circle (at 0 -10.16 270) (size 1.7 1.7) (drill 1) (layers "*.Cu" "*.Mask") (remove_unused_layers no) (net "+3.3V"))
  (pad "6" thru_hole circle (at 0 -12.7 270) (size 1.7 1.7) (drill 1) (layers "*.Cu" "*.Mask") (remove_unused_layers no) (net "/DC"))
  (pad "7" thru_hole circle (at 0 -15.24 270) (size 1.7 1.7) (drill 1) (layers "*.Cu" "*.Mask") (remove_unused_layers no) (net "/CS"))
  (pad "8" thru_hole circle (at 0 -17.78 270) (size 1.7 1.7) (drill 1) (layers "*.Cu" "*.Mask") (remove_unused_layers no) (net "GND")))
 (gr_rect (start 55 29) (end 120 89) (stroke (width 0.05) (type default)) (fill no) (layer "Edge.Cuts"))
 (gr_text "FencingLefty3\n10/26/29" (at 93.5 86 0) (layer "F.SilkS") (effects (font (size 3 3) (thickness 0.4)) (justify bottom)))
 (segment (start 69.045 63.875) (end 70.22 62.7) (width 0.2) (layer "F.Cu") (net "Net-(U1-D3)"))
 (segment (start 70.22 62.7) (end 97.18 62.7) (width 0.2) (layer "F.Cu") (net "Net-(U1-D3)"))
 (segment (start 97.18 62.7) (end 110 49.88) (width 0.2) (layer "F.Cu") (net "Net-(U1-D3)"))
 (segment (start 111.062 47.789786) (end 111.062 61.102) (width 0.2) (layer "F.Cu") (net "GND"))
 (segment (start 111.062 61.102) (end 115.08 65.12) (width 0.2) (layer "F.Cu") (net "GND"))
 (segment (start 95.3 43) (end 106.272214 43) (width 0.2) (layer "F.Cu") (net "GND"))
 (segment (start 106.272214 43) (end 111.062 47.789786) (width 0.2) (layer "F.Cu") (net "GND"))
 (segment (start 62.695 66.415) (end 67.288402 66.415) (width 0.2) (layer "B.Cu") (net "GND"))
 (segment (start 80.96 73.5) (end 90 64.46) (width 0.2) (layer "B.Cu") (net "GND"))
 (segment (start 82.55 62.2) (end 112.16 62.2) (width 0.2) (layer "B.Cu") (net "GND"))
 (segment (start 90 59.15) (end 93.25 55.9) (width 0.2) (layer "B.Cu") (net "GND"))
 (segment (start 114.018 64.058) (end 115.08 65.12) (width 0.2) (layer "B.Cu") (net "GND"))
 (segment (start 78.75 58.4) (end 82.55 62.2) (width 0.2) (layer "B.Cu") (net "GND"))
 (segment (start 93.511522 63) (end 112.96 63) (width 0.2) (layer "B.Cu") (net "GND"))
 (segment (start 112.96 63) (end 115.08 65.12) (width 0.2) (layer "B.Cu") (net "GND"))
 (segment (start 98.74 73.5) (end 106.7 73.5) (width 0.2) (layer "B.Cu") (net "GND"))
 (segment (start 91.95 57.2) (end 91.95 61.438478) (width 0.2) (layer "B.Cu") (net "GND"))
 (segment (start 106.7 73.5) (end 115.08 65.12) (width 0.2) (layer "B.Cu") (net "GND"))
 (segment (start 74.373402 73.5) (end 80.96 73.5) (width 0.2) (layer "B.Cu") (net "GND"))
 (segment (start 62.69 66.41) (end 62.695 66.415) (width 0.2) (layer "B.Cu") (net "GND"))
 (segment (start 112.16 62.2) (end 115.08 65.12) (width 0.2) (layer "B.Cu") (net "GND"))
 (segment (start 93.25 55.9) (end 91.95 57.2) (width 0.2) (layer "B.Cu") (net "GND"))
 (segment (start 90 64.46) (end 90 59.15) (width 0.2) (layer "B.Cu") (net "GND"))
 (segment (start 91.95 61.438478) (end 93.511522 63) (width 0.2) (layer "B.Cu") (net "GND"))
 (segment (start 62.69 45.46) (end 62.69 66.41) (width 0.2) (layer "B.Cu") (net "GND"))
 (segment (start 67.288402 66.415) (end 74.373402 73.5) (width 0.2) (layer "B.Cu") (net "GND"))
 (segment (start 114.018 48.818) (end 115.08 49.88) (width 0.2) (layer "B.Cu") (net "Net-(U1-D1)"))
 (segment (start 85.832 48.818) (end 114.018 48.818) (width 0.2) (layer "B.Cu") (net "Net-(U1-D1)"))
 (segment (start 78.75 55.9) (end 85.832 48.818) (width 0.2) (layer "B.Cu") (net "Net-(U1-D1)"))
 (segment (start 77.45 54.6) (end 83.632 48.418) (width 0.2) (layer "B.Cu") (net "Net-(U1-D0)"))
 (segment (start 116.158 48.418) (end 117.62 49.88) (width 0.2) (layer "B.Cu") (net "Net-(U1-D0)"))
 (segment (start 78.75 60.9) (end 77.45 59.6) (width 0.2) (layer "B.Cu") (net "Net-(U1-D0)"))
 (segment (start 83.632 48.418) (end 116.158 48.418) (width 0.2) (layer "B.Cu") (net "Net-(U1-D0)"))
 (segment (start 77.45 59.6) (end 77.45 54.6) (width 0.2) (layer "B.Cu") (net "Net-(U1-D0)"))
 (segment (start 101.52 60.9) (end 112.54 49.88) (width 0.2) (layer "B.Cu") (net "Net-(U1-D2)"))
 (segment (start 93.25 60.9) (end 101.52 60.9) (width 0.2) (layer "B.Cu") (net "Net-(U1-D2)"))
 (segment (start 106.18663 47.529) (end 107.46 48.80237) (width 0.2) (layer "F.Cu") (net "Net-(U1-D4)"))
 (segment (start 73.649 47.529) (end 106.18663 47.529) (width 0.2) (layer "F.Cu") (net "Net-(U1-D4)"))
 (segment (start 69.04 42.92) (end 73.649 47.529) (width 0.2) (layer "F.Cu") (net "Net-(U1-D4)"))
 (segment (start 107.46 48.80237) (end 107.46 49.88) (width 0.2) (layer "F.Cu") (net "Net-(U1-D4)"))
 (segment (start 87.7 43) (end 91.829 47.129) (width 0.2) (layer "F.Cu") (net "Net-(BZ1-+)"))
 (segment (start 107.861214 47.129) (end 108.522 47.789786) (width 0.2) (layer "F.Cu") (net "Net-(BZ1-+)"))
 (segment (start 108.522 47.789786) (end 108.522 50.319895) (width 0.2) (layer "F.Cu") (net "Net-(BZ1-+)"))
 (segment (start 107.899895 50.942) (end 106.817 50.942) (width 0.2) (layer "F.Cu") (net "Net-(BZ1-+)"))
 (segment (start 106.817 50.942) (end 104.92 49.045) (width 0.2) (layer "F.Cu") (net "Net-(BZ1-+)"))
 (segment (start 91.829 47.129) (end 107.861214 47.129) (width 0.2) (layer "F.Cu") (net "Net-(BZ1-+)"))
 (segment (start 108.522 50.319895) (end 107.899895 50.942) (width 0.2) (layer "F.Cu") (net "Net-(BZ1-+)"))
 (segment (start 84.65 72.35) (end 89.97 72.35) (width 0.2) (layer "F.Cu") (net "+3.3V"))
 (segment (start 112.54 66.19763) (end 112.54 65.12) (width 0.2) (layer "F.Cu") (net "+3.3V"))
 (segment (start 111.23763 67.5) (end 112.54 66.19763) (width 0.2) (layer "F.Cu") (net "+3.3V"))
 (segment (start 89.97 72.35) (end 91.12 73.5) (width 0.2) (layer "F.Cu") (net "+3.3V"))
 (segment (start 83.5 73.5) (end 84.65 72.35) (width 0.2) (layer "F.Cu") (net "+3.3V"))
 (segment (start 89.5 67.5) (end 111.23763 67.5) (width 0.2) (layer "F.Cu") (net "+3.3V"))
 (segment (start 83.5 73.5) (end 89.5 67.5) (width 0.2) (layer "F.Cu") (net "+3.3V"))
 (segment (start 82.35 73.976346) (end 82.35 73.023654) (width 0.2) (layer "F.Cu") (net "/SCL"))
 (segment (start 106.398 64.058) (end 107.46 65.12) (width 0.2) (layer "F.Cu") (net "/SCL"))
 (segment (start 86.04 73.5) (end 84.89 74.65) (width 0.2) (layer "F.Cu") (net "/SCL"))
 (segment (start 84.89 74.65) (end 83.023654 74.65) (width 0.2) (layer "F.Cu") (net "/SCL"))
 (segment (start 91.315654 64.058) (end 106.398 64.058) (width 0.2) (layer "F.Cu") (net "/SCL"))
 (segment (start 83.023654 74.65) (end 82.35 73.976346) (width 0.2) (layer "F.Cu") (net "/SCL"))
 (segment (start 82.35 73.023654) (end 91.315654 64.058) (width 0.2) (layer "F.Cu") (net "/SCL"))
 (segment (start 113.602 64.680105) (end 112.979895 64.058) (width 0.2) (layer "F.Cu") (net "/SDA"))
 (segment (start 113.602 67.210214) (end 113.602 64.680105) (width 0.2) (layer "F.Cu") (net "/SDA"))
 (segment (start 111.062 64.058) (end 110 65.12) (width 0.2) (layer "F.Cu") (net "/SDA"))
 (segment (start 89.73 74.65) (end 106.162214 74.65) (width 0.2) (layer "F.Cu") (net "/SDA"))
 (segment (start 112.979895 64.058) (end 111.062 64.058) (width 0.2) (layer "F.Cu") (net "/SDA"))
 (segment (start 106.162214 74.65) (end 113.602 67.210214) (width 0.2) (layer "F.Cu") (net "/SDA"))
 (segment (start 88.58 73.5) (end 89.73 74.65) (width 0.2) (layer "F.Cu") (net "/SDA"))
 (segment (start 97.69 72.35) (end 104.92 65.12) (width 0.2) (layer "B.Cu") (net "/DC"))
 (segment (start 94.81 72.35) (end 97.69 72.35) (width 0.2) (layer "B.Cu") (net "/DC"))
 (segment (start 93.66 73.5) (end 94.81 72.35) (width 0.2) (layer "B.Cu") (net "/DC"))
 (segment (start 92.51 73.023654) (end 100.413654 65.12) (width 0.2) (layer "B.Cu") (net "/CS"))
 (segment (start 96.2 73.5) (end 95.05 74.65) (width 0.2) (layer "B.Cu") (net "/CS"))
 (segment (start 100.413654 65.12) (end 102.38 65.12) (width 0.2) (layer "B.Cu") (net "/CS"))
 (segment (start 95.05 74.65) (end 93.183654 74.65) (width 0.2) (layer "B.Cu") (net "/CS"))
 (segment (start 92.51 73.976346) (end 92.51 73.023654) (width 0.2) (layer "B.Cu") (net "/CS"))
 (segment (start 93.183654 74.65) (end 92.51 73.976346) (width 0.2) (layer "B.Cu") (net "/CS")))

